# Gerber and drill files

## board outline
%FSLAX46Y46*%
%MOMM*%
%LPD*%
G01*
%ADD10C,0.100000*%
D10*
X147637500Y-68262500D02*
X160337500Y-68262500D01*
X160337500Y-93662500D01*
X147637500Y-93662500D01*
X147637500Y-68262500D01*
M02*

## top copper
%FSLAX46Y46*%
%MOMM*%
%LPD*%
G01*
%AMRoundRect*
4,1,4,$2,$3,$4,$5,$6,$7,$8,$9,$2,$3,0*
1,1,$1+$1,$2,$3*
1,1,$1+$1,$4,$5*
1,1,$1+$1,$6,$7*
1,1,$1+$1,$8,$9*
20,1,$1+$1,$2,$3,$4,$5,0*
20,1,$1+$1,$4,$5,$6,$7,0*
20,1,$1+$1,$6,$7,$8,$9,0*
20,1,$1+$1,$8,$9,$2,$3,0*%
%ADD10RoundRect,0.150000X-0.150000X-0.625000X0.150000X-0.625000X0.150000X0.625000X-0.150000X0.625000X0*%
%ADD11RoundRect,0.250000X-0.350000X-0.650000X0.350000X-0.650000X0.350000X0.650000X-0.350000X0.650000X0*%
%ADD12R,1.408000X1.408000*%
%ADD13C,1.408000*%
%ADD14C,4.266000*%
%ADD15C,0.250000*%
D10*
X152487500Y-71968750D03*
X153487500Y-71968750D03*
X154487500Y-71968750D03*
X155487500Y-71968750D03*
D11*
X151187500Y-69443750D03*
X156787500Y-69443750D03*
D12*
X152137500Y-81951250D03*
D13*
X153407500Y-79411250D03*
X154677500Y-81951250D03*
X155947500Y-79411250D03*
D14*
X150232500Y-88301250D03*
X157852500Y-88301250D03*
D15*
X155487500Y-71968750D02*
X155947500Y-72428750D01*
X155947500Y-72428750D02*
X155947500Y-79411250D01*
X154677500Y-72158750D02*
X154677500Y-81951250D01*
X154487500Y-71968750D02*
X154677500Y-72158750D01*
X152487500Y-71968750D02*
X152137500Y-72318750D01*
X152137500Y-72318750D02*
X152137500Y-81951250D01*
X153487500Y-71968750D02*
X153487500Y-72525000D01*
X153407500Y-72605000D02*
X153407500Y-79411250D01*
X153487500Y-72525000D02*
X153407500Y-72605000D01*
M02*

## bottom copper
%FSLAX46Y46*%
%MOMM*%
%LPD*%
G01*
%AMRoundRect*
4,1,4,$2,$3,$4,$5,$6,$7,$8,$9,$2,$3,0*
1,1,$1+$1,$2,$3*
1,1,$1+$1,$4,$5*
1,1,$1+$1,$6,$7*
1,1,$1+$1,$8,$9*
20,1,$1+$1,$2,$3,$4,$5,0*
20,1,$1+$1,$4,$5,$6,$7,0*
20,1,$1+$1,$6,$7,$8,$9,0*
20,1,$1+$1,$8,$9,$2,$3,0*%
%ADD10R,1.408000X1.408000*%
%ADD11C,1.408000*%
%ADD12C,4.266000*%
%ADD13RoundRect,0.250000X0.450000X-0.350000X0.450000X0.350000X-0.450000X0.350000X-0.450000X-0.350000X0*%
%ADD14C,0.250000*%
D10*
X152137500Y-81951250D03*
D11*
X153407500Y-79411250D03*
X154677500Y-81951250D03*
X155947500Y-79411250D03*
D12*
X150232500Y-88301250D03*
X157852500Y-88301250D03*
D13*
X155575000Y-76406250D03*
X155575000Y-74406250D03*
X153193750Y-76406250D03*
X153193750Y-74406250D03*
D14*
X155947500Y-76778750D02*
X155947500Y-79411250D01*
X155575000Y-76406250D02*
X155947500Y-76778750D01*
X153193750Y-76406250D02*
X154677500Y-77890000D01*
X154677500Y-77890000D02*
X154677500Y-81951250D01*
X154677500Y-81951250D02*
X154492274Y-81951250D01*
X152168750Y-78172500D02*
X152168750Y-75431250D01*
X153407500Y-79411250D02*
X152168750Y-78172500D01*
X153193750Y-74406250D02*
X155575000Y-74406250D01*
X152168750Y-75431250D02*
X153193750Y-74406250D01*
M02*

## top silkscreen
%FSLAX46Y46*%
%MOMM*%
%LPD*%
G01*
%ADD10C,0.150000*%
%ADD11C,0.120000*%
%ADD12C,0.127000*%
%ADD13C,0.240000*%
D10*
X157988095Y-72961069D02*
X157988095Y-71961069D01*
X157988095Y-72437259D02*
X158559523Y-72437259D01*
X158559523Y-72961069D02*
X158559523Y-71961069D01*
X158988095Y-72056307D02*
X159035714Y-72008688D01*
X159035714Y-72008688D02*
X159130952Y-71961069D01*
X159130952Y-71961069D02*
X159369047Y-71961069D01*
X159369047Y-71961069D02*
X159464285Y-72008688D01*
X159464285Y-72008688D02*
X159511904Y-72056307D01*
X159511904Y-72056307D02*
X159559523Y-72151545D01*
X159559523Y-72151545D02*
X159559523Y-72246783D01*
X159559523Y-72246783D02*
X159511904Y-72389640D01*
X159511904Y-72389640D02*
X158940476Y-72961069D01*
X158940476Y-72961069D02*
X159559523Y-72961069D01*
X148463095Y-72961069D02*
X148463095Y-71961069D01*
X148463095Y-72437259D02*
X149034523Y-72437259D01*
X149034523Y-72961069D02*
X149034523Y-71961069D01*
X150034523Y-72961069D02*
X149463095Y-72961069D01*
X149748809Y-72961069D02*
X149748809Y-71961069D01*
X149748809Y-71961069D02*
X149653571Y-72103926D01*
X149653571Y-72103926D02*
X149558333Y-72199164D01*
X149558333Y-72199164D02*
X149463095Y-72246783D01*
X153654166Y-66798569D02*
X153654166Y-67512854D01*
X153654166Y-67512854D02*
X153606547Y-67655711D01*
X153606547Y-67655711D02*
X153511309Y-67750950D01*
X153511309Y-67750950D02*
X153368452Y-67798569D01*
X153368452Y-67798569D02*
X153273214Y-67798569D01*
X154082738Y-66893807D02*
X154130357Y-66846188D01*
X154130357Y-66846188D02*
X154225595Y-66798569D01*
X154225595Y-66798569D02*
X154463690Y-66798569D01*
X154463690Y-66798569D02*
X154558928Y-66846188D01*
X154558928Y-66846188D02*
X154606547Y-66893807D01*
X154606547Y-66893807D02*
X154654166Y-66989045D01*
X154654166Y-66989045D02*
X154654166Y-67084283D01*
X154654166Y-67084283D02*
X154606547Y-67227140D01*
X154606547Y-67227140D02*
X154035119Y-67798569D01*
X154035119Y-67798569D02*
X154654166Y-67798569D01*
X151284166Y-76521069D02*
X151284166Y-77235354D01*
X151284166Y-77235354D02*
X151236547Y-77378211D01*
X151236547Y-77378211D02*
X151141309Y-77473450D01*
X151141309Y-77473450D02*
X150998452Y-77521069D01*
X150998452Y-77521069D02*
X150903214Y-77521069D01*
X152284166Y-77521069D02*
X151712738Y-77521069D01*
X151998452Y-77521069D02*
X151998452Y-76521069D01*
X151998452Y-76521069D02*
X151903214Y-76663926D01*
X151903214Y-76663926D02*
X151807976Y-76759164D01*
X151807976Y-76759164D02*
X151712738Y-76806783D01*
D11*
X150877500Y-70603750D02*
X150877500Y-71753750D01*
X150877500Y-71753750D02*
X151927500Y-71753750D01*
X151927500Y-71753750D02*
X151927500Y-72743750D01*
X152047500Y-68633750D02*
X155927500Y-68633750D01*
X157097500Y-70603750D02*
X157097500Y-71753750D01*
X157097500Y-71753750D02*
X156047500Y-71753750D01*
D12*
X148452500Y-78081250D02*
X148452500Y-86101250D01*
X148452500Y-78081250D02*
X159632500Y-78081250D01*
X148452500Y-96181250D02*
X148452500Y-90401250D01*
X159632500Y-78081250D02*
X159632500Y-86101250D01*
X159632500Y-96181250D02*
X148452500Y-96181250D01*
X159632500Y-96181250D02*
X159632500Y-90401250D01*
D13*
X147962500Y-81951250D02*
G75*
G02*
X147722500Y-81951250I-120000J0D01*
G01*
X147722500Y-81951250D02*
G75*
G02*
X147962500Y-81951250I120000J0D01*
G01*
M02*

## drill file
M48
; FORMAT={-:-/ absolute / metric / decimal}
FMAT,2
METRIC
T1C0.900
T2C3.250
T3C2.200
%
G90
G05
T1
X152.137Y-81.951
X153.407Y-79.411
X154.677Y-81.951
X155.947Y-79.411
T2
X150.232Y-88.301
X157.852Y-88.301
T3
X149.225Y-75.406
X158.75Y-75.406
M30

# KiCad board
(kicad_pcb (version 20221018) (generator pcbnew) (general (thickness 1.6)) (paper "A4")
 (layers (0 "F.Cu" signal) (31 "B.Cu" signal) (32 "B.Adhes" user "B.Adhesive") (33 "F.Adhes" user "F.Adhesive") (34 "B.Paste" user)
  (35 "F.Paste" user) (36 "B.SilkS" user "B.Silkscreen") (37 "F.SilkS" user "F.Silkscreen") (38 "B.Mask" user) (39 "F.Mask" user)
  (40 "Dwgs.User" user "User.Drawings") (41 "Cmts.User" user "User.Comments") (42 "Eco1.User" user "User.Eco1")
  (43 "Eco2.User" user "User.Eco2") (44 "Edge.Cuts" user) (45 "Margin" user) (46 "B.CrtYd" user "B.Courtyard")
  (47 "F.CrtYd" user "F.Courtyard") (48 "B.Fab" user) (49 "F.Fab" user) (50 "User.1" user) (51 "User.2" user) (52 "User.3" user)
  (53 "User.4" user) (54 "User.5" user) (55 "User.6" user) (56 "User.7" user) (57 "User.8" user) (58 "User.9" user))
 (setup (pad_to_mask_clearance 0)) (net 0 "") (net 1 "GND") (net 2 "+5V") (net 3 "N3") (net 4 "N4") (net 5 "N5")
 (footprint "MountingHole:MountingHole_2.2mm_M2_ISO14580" (layer "F.Cu") (at 158.75 75.40625)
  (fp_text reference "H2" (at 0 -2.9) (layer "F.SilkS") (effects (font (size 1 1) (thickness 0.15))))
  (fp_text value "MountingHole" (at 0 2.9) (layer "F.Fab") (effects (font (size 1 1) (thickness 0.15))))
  (pad "" np_thru_hole circle (at 0 0) (size 2.2 2.2) (drill 2.2) (layers "*.Cu" "*.Mask")))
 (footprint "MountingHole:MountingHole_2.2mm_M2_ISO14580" (layer "F.Cu") (at 149.225 75.40625)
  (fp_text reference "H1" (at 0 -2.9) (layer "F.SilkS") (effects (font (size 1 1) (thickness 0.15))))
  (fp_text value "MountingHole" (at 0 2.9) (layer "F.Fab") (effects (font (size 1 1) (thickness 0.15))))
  (pad "" np_thru_hole circle (at 0 0) (size 2.2 2.2) (drill 2.2) (layers "*.Cu" "*.Mask")))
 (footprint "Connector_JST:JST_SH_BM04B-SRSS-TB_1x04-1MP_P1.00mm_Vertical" (layer "F.Cu") (at 153.9875 70.64375)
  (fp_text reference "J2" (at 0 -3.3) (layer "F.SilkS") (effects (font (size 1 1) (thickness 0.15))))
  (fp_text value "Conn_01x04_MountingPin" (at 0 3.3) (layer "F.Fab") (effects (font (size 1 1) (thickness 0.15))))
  (fp_line (start -3.11 -0.04) (end -3.11 1.11) (stroke (width 0.12) (type solid)) (layer "F.SilkS"))
  (fp_line (start -3.11 1.11) (end -2.06 1.11) (stroke (width 0.12) (type solid)) (layer "F.SilkS"))
  (fp_line (start -2.06 1.11) (end -2.06 2.1) (stroke (width 0.12) (type solid)) (layer "F.SilkS"))
  (fp_line (start -1.94 -2.01) (end 1.94 -2.01) (stroke (width 0.12) (type solid)) (layer "F.SilkS"))
  (fp_line (start 3.11 -0.04) (end 3.11 1.11) (stroke (width 0.12) (type solid)) (layer "F.SilkS"))
  (fp_line (start 3.11 1.11) (end 2.06 1.11) (stroke (width 0.12) (type solid)) (layer "F.SilkS"))
  (pad "1" smd roundrect (at -1.5 1.325) (size 0.6 1.55) (layers "F.Cu" "F.Paste" "F.Mask") (roundrect_rratio 0.25) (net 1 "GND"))
  (pad "2" smd roundrect (at -0.5 1.325) (size 0.6 1.55) (layers "F.Cu" "F.Paste" "F.Mask") (roundrect_rratio 0.25) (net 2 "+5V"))
  (pad "3" smd roundrect (at 0.5 1.325) (size 0.6 1.55) (layers "F.Cu" "F.Paste" "F.Mask") (roundrect_rratio 0.25) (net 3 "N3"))
  (pad "4" smd roundrect (at 1.5 1.325) (size 0.6 1.55) (layers "F.Cu" "F.Paste" "F.Mask") (roundrect_rratio 0.25) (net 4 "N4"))
  (pad "MP" smd roundrect (at -2.8 -1.2) (size 1.2 1.8) (layers "F.Cu" "F.Paste" "F.Mask") (roundrect_rratio 0.208333) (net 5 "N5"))
  (pad "MP" smd roundrect (at 2.8 -1.2) (size 1.2 1.8) (layers "F.Cu" "F.Paste" "F.Mask") (roundrect_rratio 0.208333) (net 5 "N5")))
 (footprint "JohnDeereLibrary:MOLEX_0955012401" (layer "F.Cu") (at 154.0425 88.30125)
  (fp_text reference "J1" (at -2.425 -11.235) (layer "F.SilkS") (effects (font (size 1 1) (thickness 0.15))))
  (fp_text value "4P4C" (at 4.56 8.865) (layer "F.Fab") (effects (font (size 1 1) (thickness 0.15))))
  (fp_line (start -5.59 -10.22) (end -5.59 -2.2) (stroke (width 0.127) (type solid)) (layer "F.SilkS"))
  (fp_line (start -5.59 -10.22) (end 5.59 -10.22) (stroke (width 0.127) (type solid)) (layer "F.SilkS"))
  (fp_line (start -5.59 7.88) (end -5.59 2.1) (stroke (width 0.127) (type solid)) (layer "F.SilkS"))
  (fp_line (start 5.59 -10.22) (end 5.59 -2.2) (stroke (width 0.127) (type solid)) (layer "F.SilkS"))
  (fp_line (start 5.59 7.88) (end -5.59 7.88) (stroke (width 0.127) (type solid)) (layer "F.SilkS"))
  (fp_line (start 5.59 7.88) (end 5.59 2.1) (stroke (width 0.127) (type solid)) (layer "F.SilkS"))
  (fp_circle (center -6.2 -6.35) (end -6.08 -6.35) (stroke (width 0.24) (type solid)) (fill none) (layer "F.SilkS"))
  (pad "1" thru_hole rect (at -1.905 -6.35) (size 1.408 1.408) (drill 0.9) (layers "*.Cu" "*.Mask") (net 1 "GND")
   (solder_mask_margin 0.0762))
  (pad "2" thru_hole circle (at -0.635 -8.89) (size 1.408 1.408) (drill 0.9) (layers "*.Cu" "*.Mask") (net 2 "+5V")
   (solder_mask_margin 0.0762))
  (pad "3" thru_hole circle (at 0.635 -6.35) (size 1.408 1.408) (drill 0.9) (layers "*.Cu" "*.Mask") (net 3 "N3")
   (solder_mask_margin 0.0762))
  (pad "4" thru_hole circle (at 1.905 -8.89) (size 1.408 1.408) (drill 0.9) (layers "*.Cu" "*.Mask") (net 4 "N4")
   (solder_mask_margin 0.0762))
  (pad "S1" thru_hole circle (at -3.81 0) (size 4.266 4.266) (drill 3.25) (layers "*.Cu" "*.Mask") (solder_mask_margin 0.0762))
  (pad "S2" thru_hole circle (at 3.81 0) (size 4.266 4.266) (drill 3.25) (layers "*.Cu" "*.Mask") (solder_mask_margin 0.0762)))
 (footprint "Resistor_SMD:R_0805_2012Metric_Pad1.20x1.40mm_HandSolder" (layer "B.Cu") (at 155.575 75.40625 90)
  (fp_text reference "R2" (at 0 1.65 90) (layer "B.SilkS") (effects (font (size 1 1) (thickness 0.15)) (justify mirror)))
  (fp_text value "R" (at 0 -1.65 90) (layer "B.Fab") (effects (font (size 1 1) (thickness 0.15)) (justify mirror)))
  (pad "1" smd roundrect (at -1 0 90) (size 1.2 1.4) (layers "B.Cu" "B.Paste" "B.Mask") (roundrect_rratio 0.208333) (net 4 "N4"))
  (pad "2" smd roundrect (at 1 0 90) (size 1.2 1.4) (layers "B.Cu" "B.Paste" "B.Mask") (roundrect_rratio 0.208333) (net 2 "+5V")))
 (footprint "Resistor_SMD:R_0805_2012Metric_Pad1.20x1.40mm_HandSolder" (layer "B.Cu") (at 153.19375 75.40625 90)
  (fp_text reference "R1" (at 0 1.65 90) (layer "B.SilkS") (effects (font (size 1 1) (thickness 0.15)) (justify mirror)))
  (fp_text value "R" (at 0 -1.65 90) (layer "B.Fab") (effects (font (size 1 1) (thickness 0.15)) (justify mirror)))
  (pad "1" smd roundrect (at -1 0 90) (size 1.2 1.4) (layers "B.Cu" "B.Paste" "B.Mask") (roundrect_rratio 0.208333) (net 3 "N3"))
  (pad "2" smd roundrect (at 1 0 90) (size 1.2 1.4) (layers "B.Cu" "B.Paste" "B.Mask") (roundrect_rratio 0.208333) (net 2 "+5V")))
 (gr_rect (start 147.6375 68.2625) (end 160.3375 93.6625) (stroke (width 0.1) (type default)) (fill none) (layer "Edge.Cuts"))
 (segment (start 155.4875 71.96875) (end 155.9475 72.42875) (width 0.25) (layer "F.Cu") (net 4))
 (segment (start 155.9475 72.42875) (end 155.9475 79.41125) (width 0.25) (layer "F.Cu") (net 4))
 (segment (start 155.9475 76.77875) (end 155.9475 79.41125) (width 0.25) (layer "B.Cu") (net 4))
 (segment (start 155.575 76.40625) (end 155.9475 76.77875) (width 0.25) (layer "B.Cu") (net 4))
 (segment (start 154.6775 72.15875) (end 154.6775 81.95125) (width 0.25) (layer "F.Cu") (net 3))
 (segment (start 154.4875 71.96875) (end 154.6775 72.15875) (width 0.25) (layer "F.Cu") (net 3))
 (segment (start 153.19375 76.40625) (end 154.6775 77.89) (width 0.25) (layer "B.Cu") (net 3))
 (segment (start 154.6775 77.89) (end 154.6775 81.95125) (width 0.25) (layer "B.Cu") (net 3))
 (segment (start 154.6775 81.95125) (end 154.492274 81.95125) (width 0.25) (layer "B.Cu") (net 3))
 (segment (start 152.4875 71.96875) (end 152.1375 72.31875) (width 0.25) (layer "F.Cu") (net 1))
 (segment (start 152.1375 72.31875) (end 152.1375 81.95125) (width 0.25) (layer "F.Cu") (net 1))
 (segment (start 153.4875 71.96875) (end 153.4875 72.525) (width 0.25) (layer "F.Cu") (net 2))
 (segment (start 153.4075 72.605) (end 153.4075 79.41125) (width 0.25) (layer "F.Cu") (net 2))
 (segment (start 153.4875 72.525) (end 153.4075 72.605) (width 0.25) (layer "F.Cu") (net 2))
 (segment (start 152.16875 78.1725) (end 152.16875 75.43125) (width 0.25) (layer "B.Cu") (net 2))
 (segment (start 153.4075 79.41125) (end 152.16875 78.1725) (width 0.25) (layer "B.Cu") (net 2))
 (segment (start 153.19375 74.40625) (end 155.575 74.40625) (width 0.25) (layer "B.Cu") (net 2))
 (segment (start 152.16875 75.43125) (end 153.19375 74.40625) (width 0.25) (layer "B.Cu") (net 2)))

